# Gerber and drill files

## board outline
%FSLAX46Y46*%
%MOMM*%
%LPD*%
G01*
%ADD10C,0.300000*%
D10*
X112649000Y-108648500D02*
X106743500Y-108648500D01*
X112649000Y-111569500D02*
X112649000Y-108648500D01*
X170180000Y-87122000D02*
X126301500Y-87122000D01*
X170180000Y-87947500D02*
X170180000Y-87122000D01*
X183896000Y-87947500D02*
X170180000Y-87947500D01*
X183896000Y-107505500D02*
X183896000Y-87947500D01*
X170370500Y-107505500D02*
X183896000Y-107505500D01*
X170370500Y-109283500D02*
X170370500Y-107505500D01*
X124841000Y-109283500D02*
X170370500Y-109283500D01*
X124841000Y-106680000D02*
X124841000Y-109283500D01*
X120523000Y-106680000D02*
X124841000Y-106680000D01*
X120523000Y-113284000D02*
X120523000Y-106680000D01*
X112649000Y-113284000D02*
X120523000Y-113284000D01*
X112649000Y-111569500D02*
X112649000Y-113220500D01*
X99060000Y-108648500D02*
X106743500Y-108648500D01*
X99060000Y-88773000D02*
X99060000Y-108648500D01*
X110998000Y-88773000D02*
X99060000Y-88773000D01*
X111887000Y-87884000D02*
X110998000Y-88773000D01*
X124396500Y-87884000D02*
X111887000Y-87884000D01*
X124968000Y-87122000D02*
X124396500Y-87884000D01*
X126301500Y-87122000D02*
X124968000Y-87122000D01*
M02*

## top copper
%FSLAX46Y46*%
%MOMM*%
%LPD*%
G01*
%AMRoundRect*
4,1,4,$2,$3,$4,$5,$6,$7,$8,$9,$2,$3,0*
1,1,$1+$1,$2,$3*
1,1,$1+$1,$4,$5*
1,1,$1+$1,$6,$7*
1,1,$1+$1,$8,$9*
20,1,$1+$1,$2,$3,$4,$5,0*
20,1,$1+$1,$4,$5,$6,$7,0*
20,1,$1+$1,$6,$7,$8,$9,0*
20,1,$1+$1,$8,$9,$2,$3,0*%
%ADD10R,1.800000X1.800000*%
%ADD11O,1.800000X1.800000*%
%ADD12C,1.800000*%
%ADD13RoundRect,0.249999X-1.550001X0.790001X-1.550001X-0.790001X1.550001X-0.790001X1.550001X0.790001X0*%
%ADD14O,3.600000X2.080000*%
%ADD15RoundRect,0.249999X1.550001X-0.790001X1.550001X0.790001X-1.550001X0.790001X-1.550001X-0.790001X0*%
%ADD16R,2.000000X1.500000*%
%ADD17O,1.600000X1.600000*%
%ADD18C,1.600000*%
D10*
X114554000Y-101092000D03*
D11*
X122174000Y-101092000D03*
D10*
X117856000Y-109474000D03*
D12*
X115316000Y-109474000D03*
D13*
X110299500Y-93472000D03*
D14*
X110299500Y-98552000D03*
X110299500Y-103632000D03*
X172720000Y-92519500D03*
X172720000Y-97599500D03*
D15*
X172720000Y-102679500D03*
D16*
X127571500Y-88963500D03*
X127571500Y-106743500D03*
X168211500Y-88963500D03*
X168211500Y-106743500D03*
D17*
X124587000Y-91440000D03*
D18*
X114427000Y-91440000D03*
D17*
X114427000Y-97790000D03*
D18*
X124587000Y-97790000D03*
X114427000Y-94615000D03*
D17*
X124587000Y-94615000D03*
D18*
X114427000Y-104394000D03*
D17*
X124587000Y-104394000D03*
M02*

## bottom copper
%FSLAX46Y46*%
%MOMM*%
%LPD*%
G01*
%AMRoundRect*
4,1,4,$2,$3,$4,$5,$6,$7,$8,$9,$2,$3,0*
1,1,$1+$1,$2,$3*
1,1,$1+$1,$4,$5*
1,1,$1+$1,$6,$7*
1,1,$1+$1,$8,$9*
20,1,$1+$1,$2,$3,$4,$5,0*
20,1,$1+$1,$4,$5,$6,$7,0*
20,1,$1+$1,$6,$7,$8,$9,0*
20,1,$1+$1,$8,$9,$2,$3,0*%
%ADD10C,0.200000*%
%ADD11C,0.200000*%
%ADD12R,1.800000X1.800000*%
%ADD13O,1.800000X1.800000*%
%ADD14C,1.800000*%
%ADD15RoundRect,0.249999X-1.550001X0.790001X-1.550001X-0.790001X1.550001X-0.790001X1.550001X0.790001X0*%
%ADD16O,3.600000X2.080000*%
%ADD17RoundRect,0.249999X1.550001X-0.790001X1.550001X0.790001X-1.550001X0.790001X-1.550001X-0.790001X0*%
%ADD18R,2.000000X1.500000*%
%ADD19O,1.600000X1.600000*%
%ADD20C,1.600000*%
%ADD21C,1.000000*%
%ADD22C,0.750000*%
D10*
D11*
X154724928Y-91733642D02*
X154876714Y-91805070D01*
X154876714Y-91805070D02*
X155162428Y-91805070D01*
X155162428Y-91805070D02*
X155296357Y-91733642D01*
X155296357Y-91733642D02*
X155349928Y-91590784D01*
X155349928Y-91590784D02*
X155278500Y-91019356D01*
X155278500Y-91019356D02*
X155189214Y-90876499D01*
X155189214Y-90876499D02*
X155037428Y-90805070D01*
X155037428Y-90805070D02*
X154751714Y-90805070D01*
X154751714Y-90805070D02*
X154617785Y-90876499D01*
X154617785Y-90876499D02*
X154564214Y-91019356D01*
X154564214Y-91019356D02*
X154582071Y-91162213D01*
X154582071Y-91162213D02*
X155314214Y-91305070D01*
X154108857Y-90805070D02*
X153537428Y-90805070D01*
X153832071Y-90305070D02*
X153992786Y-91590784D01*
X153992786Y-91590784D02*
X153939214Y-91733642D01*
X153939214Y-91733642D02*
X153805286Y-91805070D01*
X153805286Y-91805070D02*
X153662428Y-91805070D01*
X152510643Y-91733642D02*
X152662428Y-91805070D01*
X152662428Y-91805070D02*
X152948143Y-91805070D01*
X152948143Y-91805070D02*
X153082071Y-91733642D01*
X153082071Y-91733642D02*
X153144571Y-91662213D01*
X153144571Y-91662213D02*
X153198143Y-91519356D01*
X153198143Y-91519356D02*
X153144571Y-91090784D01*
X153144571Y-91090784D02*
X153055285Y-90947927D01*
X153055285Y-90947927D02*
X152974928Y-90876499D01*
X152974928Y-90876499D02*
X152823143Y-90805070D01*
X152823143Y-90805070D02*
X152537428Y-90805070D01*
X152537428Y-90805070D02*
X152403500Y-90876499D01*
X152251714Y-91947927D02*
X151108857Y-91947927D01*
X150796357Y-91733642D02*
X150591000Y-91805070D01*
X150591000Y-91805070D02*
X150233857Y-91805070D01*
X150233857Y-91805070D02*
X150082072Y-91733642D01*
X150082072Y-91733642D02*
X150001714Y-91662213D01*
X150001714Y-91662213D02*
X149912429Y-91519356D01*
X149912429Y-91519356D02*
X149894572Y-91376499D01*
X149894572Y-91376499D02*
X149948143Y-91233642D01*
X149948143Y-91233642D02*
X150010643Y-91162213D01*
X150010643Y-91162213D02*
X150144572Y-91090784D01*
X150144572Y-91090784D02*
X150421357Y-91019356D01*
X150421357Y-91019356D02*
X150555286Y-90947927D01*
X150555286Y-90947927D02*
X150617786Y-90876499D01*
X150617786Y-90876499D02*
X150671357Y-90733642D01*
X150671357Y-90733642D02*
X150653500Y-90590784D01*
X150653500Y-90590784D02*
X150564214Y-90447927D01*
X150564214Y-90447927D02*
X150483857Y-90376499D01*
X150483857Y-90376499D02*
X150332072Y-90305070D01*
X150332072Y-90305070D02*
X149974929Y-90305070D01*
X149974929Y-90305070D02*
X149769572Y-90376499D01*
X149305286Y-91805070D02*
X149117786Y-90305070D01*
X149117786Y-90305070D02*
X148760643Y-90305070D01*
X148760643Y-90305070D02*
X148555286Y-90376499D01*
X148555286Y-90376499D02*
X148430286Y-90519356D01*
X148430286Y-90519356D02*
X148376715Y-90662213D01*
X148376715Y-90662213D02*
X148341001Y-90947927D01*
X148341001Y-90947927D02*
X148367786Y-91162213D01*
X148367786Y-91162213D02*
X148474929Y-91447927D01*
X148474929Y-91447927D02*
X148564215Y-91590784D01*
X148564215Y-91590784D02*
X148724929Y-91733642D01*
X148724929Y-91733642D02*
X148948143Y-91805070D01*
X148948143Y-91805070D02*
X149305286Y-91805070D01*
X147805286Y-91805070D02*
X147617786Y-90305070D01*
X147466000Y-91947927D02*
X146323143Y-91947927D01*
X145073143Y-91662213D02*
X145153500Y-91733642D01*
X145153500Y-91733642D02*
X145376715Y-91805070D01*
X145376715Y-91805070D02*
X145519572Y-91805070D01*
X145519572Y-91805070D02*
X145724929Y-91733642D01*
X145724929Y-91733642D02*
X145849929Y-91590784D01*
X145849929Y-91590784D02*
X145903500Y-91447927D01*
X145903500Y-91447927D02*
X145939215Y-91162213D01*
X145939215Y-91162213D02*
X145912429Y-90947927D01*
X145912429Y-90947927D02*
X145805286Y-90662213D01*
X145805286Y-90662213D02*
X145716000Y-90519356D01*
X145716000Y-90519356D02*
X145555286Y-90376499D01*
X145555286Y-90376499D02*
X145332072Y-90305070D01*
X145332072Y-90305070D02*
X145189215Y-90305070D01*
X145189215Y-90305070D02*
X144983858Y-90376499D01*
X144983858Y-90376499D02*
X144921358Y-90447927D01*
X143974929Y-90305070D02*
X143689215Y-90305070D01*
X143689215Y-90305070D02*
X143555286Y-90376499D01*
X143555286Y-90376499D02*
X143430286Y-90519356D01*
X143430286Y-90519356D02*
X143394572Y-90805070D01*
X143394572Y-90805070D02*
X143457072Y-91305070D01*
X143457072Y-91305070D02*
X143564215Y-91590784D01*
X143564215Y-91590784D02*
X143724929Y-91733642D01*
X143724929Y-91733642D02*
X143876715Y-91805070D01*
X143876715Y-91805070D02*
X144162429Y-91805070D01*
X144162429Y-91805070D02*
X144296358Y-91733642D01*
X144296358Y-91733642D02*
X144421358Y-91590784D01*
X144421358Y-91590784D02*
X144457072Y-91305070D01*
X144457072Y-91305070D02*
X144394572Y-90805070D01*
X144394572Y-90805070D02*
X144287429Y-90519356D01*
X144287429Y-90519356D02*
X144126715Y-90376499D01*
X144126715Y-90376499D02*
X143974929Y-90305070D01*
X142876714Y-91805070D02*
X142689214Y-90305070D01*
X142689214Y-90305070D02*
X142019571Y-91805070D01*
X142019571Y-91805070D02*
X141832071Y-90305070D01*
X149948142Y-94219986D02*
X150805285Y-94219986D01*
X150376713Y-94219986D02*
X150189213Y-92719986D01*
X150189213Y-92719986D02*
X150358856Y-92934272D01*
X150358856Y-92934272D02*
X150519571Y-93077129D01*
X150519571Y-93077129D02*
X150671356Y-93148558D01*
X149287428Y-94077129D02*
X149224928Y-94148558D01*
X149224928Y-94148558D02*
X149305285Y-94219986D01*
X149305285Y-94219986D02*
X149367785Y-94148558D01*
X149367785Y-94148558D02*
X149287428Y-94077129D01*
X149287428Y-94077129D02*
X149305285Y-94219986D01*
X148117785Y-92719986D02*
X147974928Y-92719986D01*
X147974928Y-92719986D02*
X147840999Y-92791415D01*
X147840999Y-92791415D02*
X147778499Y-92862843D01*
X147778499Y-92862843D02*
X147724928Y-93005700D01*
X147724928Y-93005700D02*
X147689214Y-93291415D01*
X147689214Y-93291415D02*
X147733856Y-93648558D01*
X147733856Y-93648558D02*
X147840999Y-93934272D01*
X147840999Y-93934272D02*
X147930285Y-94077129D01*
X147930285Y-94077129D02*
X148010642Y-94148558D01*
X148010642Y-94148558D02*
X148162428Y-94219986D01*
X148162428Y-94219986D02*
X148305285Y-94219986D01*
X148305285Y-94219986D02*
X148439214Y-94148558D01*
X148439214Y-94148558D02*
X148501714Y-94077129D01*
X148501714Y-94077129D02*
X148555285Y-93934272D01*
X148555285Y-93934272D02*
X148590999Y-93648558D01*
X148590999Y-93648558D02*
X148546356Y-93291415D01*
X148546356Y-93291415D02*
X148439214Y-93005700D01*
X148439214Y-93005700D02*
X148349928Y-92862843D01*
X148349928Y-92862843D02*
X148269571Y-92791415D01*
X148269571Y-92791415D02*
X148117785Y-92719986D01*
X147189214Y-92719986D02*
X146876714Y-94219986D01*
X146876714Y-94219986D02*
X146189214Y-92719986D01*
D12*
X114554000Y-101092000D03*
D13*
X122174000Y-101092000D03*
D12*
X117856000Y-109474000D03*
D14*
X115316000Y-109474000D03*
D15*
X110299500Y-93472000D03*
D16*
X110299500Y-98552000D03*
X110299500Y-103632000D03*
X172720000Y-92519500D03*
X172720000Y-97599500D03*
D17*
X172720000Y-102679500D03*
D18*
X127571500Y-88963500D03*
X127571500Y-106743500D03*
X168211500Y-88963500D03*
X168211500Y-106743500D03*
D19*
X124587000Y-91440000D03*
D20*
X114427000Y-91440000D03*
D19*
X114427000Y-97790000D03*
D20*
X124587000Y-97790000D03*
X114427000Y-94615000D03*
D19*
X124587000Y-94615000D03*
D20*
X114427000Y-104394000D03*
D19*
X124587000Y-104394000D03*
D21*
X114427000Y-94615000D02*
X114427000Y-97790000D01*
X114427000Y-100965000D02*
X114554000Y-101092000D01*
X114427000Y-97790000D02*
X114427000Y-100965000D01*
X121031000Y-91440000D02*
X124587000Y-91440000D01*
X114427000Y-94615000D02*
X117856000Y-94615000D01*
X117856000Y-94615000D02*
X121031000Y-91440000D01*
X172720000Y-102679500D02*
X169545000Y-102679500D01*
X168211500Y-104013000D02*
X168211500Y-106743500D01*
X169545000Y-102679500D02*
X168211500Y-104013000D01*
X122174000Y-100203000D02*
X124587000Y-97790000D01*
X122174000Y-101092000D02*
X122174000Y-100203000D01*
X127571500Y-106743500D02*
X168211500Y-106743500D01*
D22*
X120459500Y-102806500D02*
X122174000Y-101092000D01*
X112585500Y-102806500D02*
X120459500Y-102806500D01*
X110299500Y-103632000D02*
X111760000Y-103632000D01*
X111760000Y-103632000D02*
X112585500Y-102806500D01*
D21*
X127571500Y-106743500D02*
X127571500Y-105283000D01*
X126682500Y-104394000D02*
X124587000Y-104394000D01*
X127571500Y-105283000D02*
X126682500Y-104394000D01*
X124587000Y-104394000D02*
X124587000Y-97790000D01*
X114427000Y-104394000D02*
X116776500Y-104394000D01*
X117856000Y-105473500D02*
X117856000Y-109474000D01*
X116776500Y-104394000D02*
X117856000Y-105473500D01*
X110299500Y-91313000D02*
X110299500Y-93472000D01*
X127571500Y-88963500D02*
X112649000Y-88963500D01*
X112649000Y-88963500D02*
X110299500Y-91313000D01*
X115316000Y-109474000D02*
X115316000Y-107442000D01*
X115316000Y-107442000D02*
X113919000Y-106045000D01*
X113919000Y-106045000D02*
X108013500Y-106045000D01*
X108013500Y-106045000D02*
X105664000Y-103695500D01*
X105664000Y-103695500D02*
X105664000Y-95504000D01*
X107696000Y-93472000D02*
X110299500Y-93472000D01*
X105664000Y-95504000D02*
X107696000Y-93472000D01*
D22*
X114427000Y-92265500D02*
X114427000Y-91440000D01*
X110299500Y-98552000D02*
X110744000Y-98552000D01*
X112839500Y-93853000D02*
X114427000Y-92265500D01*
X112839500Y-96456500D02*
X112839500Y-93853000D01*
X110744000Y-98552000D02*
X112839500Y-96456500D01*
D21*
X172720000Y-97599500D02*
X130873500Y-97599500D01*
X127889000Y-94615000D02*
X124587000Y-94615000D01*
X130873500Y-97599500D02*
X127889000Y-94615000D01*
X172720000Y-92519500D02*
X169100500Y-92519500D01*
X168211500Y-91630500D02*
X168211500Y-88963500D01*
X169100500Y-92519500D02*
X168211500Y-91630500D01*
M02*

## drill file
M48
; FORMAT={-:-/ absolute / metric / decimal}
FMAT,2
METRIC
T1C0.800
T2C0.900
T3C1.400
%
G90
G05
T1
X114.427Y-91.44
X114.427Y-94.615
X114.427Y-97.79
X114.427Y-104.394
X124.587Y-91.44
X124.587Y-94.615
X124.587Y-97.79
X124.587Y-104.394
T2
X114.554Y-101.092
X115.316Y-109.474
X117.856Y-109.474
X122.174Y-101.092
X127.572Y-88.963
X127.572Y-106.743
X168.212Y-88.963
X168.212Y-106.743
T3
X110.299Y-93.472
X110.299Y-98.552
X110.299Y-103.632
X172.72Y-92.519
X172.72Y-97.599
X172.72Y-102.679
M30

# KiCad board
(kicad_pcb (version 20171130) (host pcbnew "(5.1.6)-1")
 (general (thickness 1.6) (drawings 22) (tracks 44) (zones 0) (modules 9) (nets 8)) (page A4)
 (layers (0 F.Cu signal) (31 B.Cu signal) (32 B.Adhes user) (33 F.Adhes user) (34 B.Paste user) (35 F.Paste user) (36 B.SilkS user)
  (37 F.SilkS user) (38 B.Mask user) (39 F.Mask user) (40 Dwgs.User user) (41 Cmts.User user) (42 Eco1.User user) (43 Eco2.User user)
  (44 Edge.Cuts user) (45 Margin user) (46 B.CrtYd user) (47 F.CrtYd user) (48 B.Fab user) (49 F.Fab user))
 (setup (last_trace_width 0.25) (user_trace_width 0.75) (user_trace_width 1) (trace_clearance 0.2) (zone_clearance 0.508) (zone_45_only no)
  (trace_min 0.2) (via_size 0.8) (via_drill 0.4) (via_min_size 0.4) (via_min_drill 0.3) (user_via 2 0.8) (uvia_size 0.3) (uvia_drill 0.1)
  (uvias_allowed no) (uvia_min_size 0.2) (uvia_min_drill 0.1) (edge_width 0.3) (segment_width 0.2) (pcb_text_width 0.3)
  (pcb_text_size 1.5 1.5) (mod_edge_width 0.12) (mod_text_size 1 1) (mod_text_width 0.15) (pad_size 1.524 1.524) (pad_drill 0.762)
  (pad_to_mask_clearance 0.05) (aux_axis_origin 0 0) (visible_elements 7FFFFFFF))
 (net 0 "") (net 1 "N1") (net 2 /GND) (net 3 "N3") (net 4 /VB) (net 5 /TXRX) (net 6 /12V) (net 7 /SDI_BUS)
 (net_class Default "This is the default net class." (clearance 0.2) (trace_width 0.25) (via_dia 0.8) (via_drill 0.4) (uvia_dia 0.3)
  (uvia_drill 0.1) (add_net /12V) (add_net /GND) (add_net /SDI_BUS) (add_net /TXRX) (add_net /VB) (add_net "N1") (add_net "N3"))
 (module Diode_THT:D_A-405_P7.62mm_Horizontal (layer F.Cu) (at 114.554 101.092)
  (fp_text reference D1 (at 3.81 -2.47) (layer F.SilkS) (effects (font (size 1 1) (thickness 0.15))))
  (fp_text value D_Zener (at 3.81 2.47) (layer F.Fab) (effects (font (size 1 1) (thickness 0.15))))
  (pad 1 thru_hole rect (at 0 0) (size 1.8 1.8) (drill 0.9) (layers *.Cu *.Mask) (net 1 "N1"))
  (pad 2 thru_hole oval (at 7.62 0) (size 1.8 1.8) (drill 0.9) (layers *.Cu *.Mask) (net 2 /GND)))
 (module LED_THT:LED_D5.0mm (layer F.Cu) (at 117.856 109.474 180)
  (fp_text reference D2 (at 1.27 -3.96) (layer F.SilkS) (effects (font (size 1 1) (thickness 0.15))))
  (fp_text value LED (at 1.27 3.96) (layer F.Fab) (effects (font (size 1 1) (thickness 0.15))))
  (pad 1 thru_hole rect (at 0 0 180) (size 1.8 1.8) (drill 0.9) (layers *.Cu *.Mask) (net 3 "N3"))
  (pad 2 thru_hole circle (at 2.54 0 180) (size 1.8 1.8) (drill 0.9) (layers *.Cu *.Mask) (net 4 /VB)))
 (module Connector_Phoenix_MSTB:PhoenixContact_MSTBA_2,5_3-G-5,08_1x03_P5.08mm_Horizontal (layer F.Cu) (at 110.2995 93.472 270)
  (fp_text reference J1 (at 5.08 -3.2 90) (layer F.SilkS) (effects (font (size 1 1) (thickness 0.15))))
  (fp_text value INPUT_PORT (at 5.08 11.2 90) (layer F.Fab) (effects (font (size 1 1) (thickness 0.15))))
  (pad 1 thru_hole roundrect (at 0 0 270) (size 2.08 3.6) (drill 1.4) (layers *.Cu *.Mask) (roundrect_rratio 0.120192) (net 4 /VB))
  (pad 2 thru_hole oval (at 5.08 0 270) (size 2.08 3.6) (drill 1.4) (layers *.Cu *.Mask) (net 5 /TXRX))
  (pad 3 thru_hole oval (at 10.16 0 270) (size 2.08 3.6) (drill 1.4) (layers *.Cu *.Mask) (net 2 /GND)))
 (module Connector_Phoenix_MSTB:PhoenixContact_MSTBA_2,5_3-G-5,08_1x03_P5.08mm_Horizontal (layer F.Cu) (at 172.72 102.6795 90)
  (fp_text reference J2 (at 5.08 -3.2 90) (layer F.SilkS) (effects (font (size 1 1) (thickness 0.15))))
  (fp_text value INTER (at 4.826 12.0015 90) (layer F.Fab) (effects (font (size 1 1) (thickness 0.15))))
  (pad 3 thru_hole oval (at 10.16 0 90) (size 2.08 3.6) (drill 1.4) (layers *.Cu *.Mask) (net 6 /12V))
  (pad 2 thru_hole oval (at 5.08 0 90) (size 2.08 3.6) (drill 1.4) (layers *.Cu *.Mask) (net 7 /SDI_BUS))
  (pad 1 thru_hole roundrect (at 0 0 90) (size 2.08 3.6) (drill 1.4) (layers *.Cu *.Mask) (roundrect_rratio 0.120192) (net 2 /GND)))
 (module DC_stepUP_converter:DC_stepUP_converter (layer F.Cu) (at 147.8915 82.6135)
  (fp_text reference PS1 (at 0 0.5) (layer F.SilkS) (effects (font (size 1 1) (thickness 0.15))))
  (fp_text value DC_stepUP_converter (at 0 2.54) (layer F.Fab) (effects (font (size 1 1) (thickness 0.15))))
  (pad 1 thru_hole rect (at -20.32 6.35) (size 2 1.5) (drill 0.9) (layers *.Cu *.Mask) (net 4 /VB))
  (pad 2 thru_hole rect (at -20.32 24.13) (size 2 1.5) (drill 0.9) (layers *.Cu *.Mask) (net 2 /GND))
  (pad 3 thru_hole rect (at 20.32 6.35) (size 2 1.5) (drill 0.9) (layers *.Cu *.Mask) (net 6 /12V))
  (pad 4 thru_hole rect (at 20.32 24.13) (size 2 1.5) (drill 0.9) (layers *.Cu *.Mask) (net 2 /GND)))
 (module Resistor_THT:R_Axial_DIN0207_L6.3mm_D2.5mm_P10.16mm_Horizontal (layer F.Cu) (at 114.427 91.44)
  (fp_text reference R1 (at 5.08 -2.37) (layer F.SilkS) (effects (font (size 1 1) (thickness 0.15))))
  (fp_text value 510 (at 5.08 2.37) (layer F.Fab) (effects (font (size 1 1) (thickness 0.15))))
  (pad 2 thru_hole oval (at 10.16 0) (size 1.6 1.6) (drill 0.8) (layers *.Cu *.Mask) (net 1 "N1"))
  (pad 1 thru_hole circle (at 0 0) (size 1.6 1.6) (drill 0.8) (layers *.Cu *.Mask) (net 5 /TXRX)))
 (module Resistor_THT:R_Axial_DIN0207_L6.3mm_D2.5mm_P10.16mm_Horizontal (layer F.Cu) (at 124.587 97.79 180)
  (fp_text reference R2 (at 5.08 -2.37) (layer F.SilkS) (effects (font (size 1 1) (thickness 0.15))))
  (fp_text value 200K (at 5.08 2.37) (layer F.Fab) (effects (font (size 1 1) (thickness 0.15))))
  (pad 2 thru_hole oval (at 10.16 0 180) (size 1.6 1.6) (drill 0.8) (layers *.Cu *.Mask) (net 1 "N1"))
  (pad 1 thru_hole circle (at 0 0 180) (size 1.6 1.6) (drill 0.8) (layers *.Cu *.Mask) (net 2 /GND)))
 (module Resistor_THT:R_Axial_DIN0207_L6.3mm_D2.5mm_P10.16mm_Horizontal (layer F.Cu) (at 114.427 94.615)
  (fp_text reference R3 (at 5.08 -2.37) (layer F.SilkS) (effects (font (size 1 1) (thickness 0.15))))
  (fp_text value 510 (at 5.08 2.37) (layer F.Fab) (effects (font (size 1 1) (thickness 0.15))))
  (pad 1 thru_hole circle (at 0 0) (size 1.6 1.6) (drill 0.8) (layers *.Cu *.Mask) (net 1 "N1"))
  (pad 2 thru_hole oval (at 10.16 0) (size 1.6 1.6) (drill 0.8) (layers *.Cu *.Mask) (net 7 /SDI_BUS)))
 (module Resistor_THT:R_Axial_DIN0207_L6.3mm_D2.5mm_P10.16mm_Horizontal (layer F.Cu) (at 114.427 104.394)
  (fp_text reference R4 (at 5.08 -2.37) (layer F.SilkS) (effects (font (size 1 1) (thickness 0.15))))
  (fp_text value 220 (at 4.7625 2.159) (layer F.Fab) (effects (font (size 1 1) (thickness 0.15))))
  (pad 1 thru_hole circle (at 0 0) (size 1.6 1.6) (drill 0.8) (layers *.Cu *.Mask) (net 3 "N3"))
  (pad 2 thru_hole oval (at 10.16 0) (size 1.6 1.6) (drill 0.8) (layers *.Cu *.Mask) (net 2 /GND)))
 (gr_line (start 112.649 108.6485) (end 106.7435 108.6485) (layer Edge.Cuts) (width 0.3))
 (gr_line (start 112.649 111.5695) (end 112.649 108.6485) (layer Edge.Cuts) (width 0.3))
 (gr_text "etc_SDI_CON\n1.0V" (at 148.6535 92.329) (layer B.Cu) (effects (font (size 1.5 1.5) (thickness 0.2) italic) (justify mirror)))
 (gr_line (start 170.18 87.122) (end 126.3015 87.122) (layer Edge.Cuts) (width 0.3))
 (gr_line (start 170.18 87.9475) (end 170.18 87.122) (layer Edge.Cuts) (width 0.3))
 (gr_line (start 183.896 87.9475) (end 170.18 87.9475) (layer Edge.Cuts) (width 0.3))
 (gr_line (start 183.896 107.5055) (end 183.896 87.9475) (layer Edge.Cuts) (width 0.3))
 (gr_line (start 170.3705 107.5055) (end 183.896 107.5055) (layer Edge.Cuts) (width 0.3))
 (gr_line (start 170.3705 109.2835) (end 170.3705 107.5055) (layer Edge.Cuts) (width 0.3))
 (gr_line (start 124.841 109.2835) (end 170.3705 109.2835) (layer Edge.Cuts) (width 0.3))
 (gr_line (start 124.841 106.68) (end 124.841 109.2835) (layer Edge.Cuts) (width 0.3))
 (gr_line (start 120.523 106.68) (end 124.841 106.68) (layer Edge.Cuts) (width 0.3))
 (gr_line (start 120.523 113.284) (end 120.523 106.68) (layer Edge.Cuts) (width 0.3))
 (gr_line (start 112.649 113.284) (end 120.523 113.284) (layer Edge.Cuts) (width 0.3))
 (gr_line (start 112.649 111.5695) (end 112.649 113.2205) (layer Edge.Cuts) (width 0.3))
 (gr_line (start 99.06 108.6485) (end 106.7435 108.6485) (layer Edge.Cuts) (width 0.3))
 (gr_line (start 99.06 88.773) (end 99.06 108.6485) (layer Edge.Cuts) (width 0.3))
 (gr_line (start 110.998 88.773) (end 99.06 88.773) (layer Edge.Cuts) (width 0.3))
 (gr_line (start 111.887 87.884) (end 110.998 88.773) (layer Edge.Cuts) (width 0.3))
 (gr_line (start 124.3965 87.884) (end 111.887 87.884) (layer Edge.Cuts) (width 0.3))
 (gr_line (start 124.968 87.122) (end 124.3965 87.884) (layer Edge.Cuts) (width 0.3))
 (gr_line (start 126.3015 87.122) (end 124.968 87.122) (layer Edge.Cuts) (width 0.3))
 (segment (start 114.427 94.615) (end 114.427 97.79) (width 1) (layer B.Cu) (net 1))
 (segment (start 114.427 100.965) (end 114.554 101.092) (width 1) (layer B.Cu) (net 1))
 (segment (start 114.427 97.79) (end 114.427 100.965) (width 1) (layer B.Cu) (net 1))
 (segment (start 121.031 91.44) (end 124.587 91.44) (width 1) (layer B.Cu) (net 1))
 (segment (start 114.427 94.615) (end 117.856 94.615) (width 1) (layer B.Cu) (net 1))
 (segment (start 117.856 94.615) (end 121.031 91.44) (width 1) (layer B.Cu) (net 1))
 (segment (start 172.72 102.6795) (end 169.545 102.6795) (width 1) (layer B.Cu) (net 2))
 (segment (start 168.2115 104.013) (end 168.2115 106.7435) (width 1) (layer B.Cu) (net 2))
 (segment (start 169.545 102.6795) (end 168.2115 104.013) (width 1) (layer B.Cu) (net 2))
 (segment (start 122.174 100.203) (end 124.587 97.79) (width 1) (layer B.Cu) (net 2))
 (segment (start 122.174 101.092) (end 122.174 100.203) (width 1) (layer B.Cu) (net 2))
 (segment (start 127.5715 106.7435) (end 168.2115 106.7435) (width 1) (layer B.Cu) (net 2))
 (segment (start 120.4595 102.8065) (end 122.174 101.092) (width 0.75) (layer B.Cu) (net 2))
 (segment (start 112.5855 102.8065) (end 120.4595 102.8065) (width 0.75) (layer B.Cu) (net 2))
 (segment (start 110.2995 103.632) (end 111.76 103.632) (width 0.75) (layer B.Cu) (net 2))
 (segment (start 111.76 103.632) (end 112.5855 102.8065) (width 0.75) (layer B.Cu) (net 2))
 (segment (start 127.5715 106.7435) (end 127.5715 105.283) (width 1) (layer B.Cu) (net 2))
 (segment (start 126.6825 104.394) (end 124.587 104.394) (width 1) (layer B.Cu) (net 2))
 (segment (start 127.5715 105.283) (end 126.6825 104.394) (width 1) (layer B.Cu) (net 2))
 (segment (start 124.587 104.394) (end 124.587 97.79) (width 1) (layer B.Cu) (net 2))
 (segment (start 114.427 104.394) (end 116.7765 104.394) (width 1) (layer B.Cu) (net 3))
 (segment (start 117.856 105.4735) (end 117.856 109.474) (width 1) (layer B.Cu) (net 3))
 (segment (start 116.7765 104.394) (end 117.856 105.4735) (width 1) (layer B.Cu) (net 3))
 (segment (start 110.2995 91.313) (end 110.2995 93.472) (width 1) (layer B.Cu) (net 4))
 (segment (start 127.5715 88.9635) (end 112.649 88.9635) (width 1) (layer B.Cu) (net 4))
 (segment (start 112.649 88.9635) (end 110.2995 91.313) (width 1) (layer B.Cu) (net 4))
 (segment (start 115.316 109.474) (end 115.316 107.442) (width 1) (layer B.Cu) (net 4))
 (segment (start 115.316 107.442) (end 113.919 106.045) (width 1) (layer B.Cu) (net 4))
 (segment (start 113.919 106.045) (end 108.0135 106.045) (width 1) (layer B.Cu) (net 4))
 (segment (start 108.0135 106.045) (end 105.664 103.6955) (width 1) (layer B.Cu) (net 4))
 (segment (start 105.664 103.6955) (end 105.664 95.504) (width 1) (layer B.Cu) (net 4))
 (segment (start 107.696 93.472) (end 110.2995 93.472) (width 1) (layer B.Cu) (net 4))
 (segment (start 105.664 95.504) (end 107.696 93.472) (width 1) (layer B.Cu) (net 4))
 (segment (start 114.427 92.2655) (end 114.427 91.44) (width 0.75) (layer B.Cu) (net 5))
 (segment (start 110.2995 98.552) (end 110.744 98.552) (width 0.75) (layer B.Cu) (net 5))
 (segment (start 112.8395 93.853) (end 114.427 92.2655) (width 0.75) (layer B.Cu) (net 5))
 (segment (start 112.8395 96.4565) (end 112.8395 93.853) (width 0.75) (layer B.Cu) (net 5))
 (segment (start 110.744 98.552) (end 112.8395 96.4565) (width 0.75) (layer B.Cu) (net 5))
 (segment (start 172.72 97.5995) (end 130.8735 97.5995) (width 1) (layer B.Cu) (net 7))
 (segment (start 127.889 94.615) (end 124.587 94.615) (width 1) (layer B.Cu) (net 7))
 (segment (start 130.8735 97.5995) (end 127.889 94.615) (width 1) (layer B.Cu) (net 7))
 (segment (start 172.72 92.5195) (end 169.1005 92.5195) (width 1) (layer B.Cu) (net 6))
 (segment (start 168.2115 91.6305) (end 168.2115 88.9635) (width 1) (layer B.Cu) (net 6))
 (segment (start 169.1005 92.5195) (end 168.2115 91.6305) (width 1) (layer B.Cu) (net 6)))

